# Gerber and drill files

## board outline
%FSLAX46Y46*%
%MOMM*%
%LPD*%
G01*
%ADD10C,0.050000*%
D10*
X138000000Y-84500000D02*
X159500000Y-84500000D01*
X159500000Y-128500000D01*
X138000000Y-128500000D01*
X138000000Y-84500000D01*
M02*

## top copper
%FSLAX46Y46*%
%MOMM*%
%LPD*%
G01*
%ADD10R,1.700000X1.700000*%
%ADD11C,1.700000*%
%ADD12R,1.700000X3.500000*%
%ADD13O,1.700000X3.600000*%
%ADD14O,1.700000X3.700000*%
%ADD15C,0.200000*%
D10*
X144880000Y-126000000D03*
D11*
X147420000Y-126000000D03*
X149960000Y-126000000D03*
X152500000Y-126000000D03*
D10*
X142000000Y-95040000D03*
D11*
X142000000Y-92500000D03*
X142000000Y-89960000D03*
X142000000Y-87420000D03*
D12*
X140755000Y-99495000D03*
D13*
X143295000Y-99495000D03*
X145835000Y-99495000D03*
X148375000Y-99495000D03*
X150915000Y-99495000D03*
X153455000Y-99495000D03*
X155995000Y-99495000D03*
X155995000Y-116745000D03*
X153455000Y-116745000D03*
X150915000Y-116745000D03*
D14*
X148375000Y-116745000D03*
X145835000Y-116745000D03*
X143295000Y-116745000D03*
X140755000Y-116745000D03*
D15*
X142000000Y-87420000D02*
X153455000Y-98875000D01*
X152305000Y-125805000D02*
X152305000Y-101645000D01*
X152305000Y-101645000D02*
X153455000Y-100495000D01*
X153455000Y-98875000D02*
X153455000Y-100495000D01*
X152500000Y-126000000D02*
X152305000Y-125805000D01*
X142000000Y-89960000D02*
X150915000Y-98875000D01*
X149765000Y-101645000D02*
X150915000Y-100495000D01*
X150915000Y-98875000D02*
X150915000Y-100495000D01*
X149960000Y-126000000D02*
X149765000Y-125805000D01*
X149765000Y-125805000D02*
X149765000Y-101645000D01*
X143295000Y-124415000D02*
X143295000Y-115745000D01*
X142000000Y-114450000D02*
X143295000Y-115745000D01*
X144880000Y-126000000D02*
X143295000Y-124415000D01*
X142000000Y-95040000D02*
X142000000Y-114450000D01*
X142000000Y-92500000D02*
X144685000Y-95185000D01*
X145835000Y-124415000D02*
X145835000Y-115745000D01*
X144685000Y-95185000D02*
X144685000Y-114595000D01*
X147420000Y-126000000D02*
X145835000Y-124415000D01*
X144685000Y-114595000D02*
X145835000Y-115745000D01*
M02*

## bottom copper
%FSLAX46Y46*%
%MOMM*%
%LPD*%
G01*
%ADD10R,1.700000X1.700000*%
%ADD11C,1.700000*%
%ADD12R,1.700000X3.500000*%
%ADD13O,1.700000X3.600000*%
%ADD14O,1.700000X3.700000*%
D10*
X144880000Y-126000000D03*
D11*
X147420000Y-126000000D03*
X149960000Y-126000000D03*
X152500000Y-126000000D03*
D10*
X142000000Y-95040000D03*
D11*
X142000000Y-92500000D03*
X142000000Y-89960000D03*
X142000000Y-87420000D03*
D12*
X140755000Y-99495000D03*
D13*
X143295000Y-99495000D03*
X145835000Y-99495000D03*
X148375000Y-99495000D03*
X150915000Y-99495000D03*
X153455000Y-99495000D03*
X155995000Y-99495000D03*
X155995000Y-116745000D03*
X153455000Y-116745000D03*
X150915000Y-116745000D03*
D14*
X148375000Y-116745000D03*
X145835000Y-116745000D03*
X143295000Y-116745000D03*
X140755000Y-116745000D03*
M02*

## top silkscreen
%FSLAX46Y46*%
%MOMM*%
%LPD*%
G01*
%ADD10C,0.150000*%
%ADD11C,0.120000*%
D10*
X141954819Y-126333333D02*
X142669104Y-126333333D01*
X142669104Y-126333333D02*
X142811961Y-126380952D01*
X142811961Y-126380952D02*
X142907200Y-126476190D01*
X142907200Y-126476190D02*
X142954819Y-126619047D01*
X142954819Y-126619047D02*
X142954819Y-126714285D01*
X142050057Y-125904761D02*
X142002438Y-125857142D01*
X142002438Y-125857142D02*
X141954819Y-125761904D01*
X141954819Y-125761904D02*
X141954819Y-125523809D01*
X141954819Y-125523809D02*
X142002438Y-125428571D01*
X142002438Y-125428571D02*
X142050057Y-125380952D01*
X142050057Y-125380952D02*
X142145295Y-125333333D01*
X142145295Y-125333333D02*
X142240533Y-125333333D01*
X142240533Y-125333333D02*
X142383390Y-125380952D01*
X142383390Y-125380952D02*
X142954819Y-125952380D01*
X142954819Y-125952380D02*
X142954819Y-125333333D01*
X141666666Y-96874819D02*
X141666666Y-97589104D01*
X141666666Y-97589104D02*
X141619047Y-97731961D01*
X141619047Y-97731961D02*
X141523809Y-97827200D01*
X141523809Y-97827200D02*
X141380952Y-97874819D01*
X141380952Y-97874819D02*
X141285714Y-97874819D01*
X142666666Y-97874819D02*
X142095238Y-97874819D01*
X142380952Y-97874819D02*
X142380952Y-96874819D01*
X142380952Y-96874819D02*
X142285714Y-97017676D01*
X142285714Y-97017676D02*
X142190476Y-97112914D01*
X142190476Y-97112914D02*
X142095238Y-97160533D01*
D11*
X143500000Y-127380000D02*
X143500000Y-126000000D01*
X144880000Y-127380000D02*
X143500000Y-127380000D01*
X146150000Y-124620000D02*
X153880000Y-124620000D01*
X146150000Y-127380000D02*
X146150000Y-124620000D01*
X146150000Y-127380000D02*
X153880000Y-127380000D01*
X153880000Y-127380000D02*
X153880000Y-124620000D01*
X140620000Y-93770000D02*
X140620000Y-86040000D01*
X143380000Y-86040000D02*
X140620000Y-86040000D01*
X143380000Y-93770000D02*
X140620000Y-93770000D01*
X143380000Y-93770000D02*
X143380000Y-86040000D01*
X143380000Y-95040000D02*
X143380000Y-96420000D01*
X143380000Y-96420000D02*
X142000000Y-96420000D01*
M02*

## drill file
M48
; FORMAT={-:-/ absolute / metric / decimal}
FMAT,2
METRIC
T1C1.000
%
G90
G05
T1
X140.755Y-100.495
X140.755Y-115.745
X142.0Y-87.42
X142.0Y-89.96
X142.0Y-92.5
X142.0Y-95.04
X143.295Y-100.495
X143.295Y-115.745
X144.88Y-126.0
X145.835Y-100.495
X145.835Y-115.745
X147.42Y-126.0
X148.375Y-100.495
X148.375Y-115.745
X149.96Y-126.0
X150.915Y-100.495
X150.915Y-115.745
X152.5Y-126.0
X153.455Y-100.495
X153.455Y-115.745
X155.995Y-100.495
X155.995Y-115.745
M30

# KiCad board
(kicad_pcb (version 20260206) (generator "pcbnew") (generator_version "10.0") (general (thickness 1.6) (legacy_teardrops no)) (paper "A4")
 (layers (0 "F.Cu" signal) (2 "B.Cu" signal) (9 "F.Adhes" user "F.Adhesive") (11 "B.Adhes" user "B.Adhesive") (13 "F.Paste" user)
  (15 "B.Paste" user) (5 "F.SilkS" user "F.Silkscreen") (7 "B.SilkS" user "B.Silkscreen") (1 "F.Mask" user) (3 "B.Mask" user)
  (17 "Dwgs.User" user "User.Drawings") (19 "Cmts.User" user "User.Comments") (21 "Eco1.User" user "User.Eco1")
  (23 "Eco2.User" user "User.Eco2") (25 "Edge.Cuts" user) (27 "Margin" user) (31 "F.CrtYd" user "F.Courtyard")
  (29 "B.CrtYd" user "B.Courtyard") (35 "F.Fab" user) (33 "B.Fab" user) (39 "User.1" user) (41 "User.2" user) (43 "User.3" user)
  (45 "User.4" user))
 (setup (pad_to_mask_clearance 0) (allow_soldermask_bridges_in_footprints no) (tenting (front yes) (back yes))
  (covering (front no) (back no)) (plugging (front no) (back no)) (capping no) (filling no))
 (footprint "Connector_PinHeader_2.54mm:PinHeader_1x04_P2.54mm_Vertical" (layer "F.Cu") (at 144.88 126 90)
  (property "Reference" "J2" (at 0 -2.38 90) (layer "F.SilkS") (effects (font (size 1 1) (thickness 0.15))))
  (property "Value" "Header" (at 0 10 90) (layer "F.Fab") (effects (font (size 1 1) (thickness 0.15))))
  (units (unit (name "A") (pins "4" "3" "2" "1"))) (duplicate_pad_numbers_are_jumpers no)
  (fp_line (start -1.38 -1.38) (end 0 -1.38) (stroke (width 0.12) (type solid)) (layer "F.SilkS"))
  (fp_line (start -1.38 0) (end -1.38 -1.38) (stroke (width 0.12) (type solid)) (layer "F.SilkS"))
  (fp_line (start 1.38 1.27) (end 1.38 9) (stroke (width 0.12) (type solid)) (layer "F.SilkS"))
  (fp_line (start -1.38 1.27) (end 1.38 1.27) (stroke (width 0.12) (type solid)) (layer "F.SilkS"))
  (fp_line (start -1.38 1.27) (end -1.38 9) (stroke (width 0.12) (type solid)) (layer "F.SilkS"))
  (fp_line (start -1.38 9) (end 1.38 9) (stroke (width 0.12) (type solid)) (layer "F.SilkS"))
  (pad "1" thru_hole rect (at 0 0 90) (size 1.7 1.7) (drill 1) (layers "*.Cu" "*.Mask") (remove_unused_layers no) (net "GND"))
  (pad "2" thru_hole circle (at 0 2.54 90) (size 1.7 1.7) (drill 1) (layers "*.Cu" "*.Mask") (remove_unused_layers no) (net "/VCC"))
  (pad "3" thru_hole circle (at 0 5.08 90) (size 1.7 1.7) (drill 1) (layers "*.Cu" "*.Mask") (remove_unused_layers no) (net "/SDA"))
  (pad "4" thru_hole circle (at 0 7.62 90) (size 1.7 1.7) (drill 1) (layers "*.Cu" "*.Mask") (remove_unused_layers no) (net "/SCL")))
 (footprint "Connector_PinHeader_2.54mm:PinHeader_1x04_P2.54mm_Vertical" (layer "F.Cu") (at 142 95.04 180)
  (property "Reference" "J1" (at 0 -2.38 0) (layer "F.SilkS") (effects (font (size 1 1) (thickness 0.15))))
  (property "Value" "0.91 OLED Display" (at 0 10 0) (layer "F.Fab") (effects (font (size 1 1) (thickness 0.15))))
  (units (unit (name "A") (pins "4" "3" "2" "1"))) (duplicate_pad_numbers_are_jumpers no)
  (fp_line (start 1.38 1.27) (end 1.38 9) (stroke (width 0.12) (type solid)) (layer "F.SilkS"))
  (fp_line (start -1.38 9) (end 1.38 9) (stroke (width 0.12) (type solid)) (layer "F.SilkS"))
  (fp_line (start -1.38 1.27) (end 1.38 1.27) (stroke (width 0.12) (type solid)) (layer "F.SilkS"))
  (fp_line (start -1.38 1.27) (end -1.38 9) (stroke (width 0.12) (type solid)) (layer "F.SilkS"))
  (fp_line (start -1.38 0) (end -1.38 -1.38) (stroke (width 0.12) (type solid)) (layer "F.SilkS"))
  (fp_line (start -1.38 -1.38) (end 0 -1.38) (stroke (width 0.12) (type solid)) (layer "F.SilkS"))
  (pad "1" thru_hole rect (at 0 0 180) (size 1.7 1.7) (drill 1) (layers "*.Cu" "*.Mask") (remove_unused_layers no) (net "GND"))
  (pad "2" thru_hole circle (at 0 2.54 180) (size 1.7 1.7) (drill 1) (layers "*.Cu" "*.Mask") (remove_unused_layers no) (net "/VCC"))
  (pad "3" thru_hole circle (at 0 5.08 180) (size 1.7 1.7) (drill 1) (layers "*.Cu" "*.Mask") (remove_unused_layers no) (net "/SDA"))
  (pad "4" thru_hole circle (at 0 7.62 180) (size 1.7 1.7) (drill 1) (layers "*.Cu" "*.Mask") (remove_unused_layers no) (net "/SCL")))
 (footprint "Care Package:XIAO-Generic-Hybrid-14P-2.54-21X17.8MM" (layer "B.Cu") (at 148.375 108.12 -90)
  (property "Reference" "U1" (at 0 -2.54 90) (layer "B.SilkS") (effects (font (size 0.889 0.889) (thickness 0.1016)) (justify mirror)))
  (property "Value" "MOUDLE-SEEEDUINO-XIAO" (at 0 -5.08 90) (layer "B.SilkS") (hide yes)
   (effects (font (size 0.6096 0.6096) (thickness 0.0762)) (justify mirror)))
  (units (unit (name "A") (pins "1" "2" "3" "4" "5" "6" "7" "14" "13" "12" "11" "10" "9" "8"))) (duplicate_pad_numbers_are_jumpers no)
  (pad "1" thru_hole rect (at -7.625 7.62 270) (size 3.5 1.7) (drill 1 (offset -1 0)) (layers "*.Cu" "*.Mask") (remove_unused_layers no)
   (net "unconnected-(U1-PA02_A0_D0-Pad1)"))
  (pad "2" thru_hole oval (at -7.625 5.08 270) (size 3.6 1.7) (drill 1 (offset -1 0)) (layers "*.Cu" "*.Mask") (remove_unused_layers no)
   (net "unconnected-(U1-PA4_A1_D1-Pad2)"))
  (pad "3" thru_hole oval (at -7.625 2.54 270) (size 3.6 1.7) (drill 1 (offset -1 0)) (layers "*.Cu" "*.Mask") (remove_unused_layers no)
   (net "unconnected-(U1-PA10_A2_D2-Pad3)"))
  (pad "4" thru_hole oval (at -7.625 0 270) (size 3.6 1.7) (drill 1 (offset -1 0)) (layers "*.Cu" "*.Mask") (remove_unused_layers no)
   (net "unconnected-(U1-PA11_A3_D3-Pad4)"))
  (pad "5" thru_hole oval (at -7.625 -2.54 270) (size 3.6 1.7) (drill 1 (offset -1 0)) (layers "*.Cu" "*.Mask") (remove_unused_layers no)
   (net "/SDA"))
  (pad "6" thru_hole oval (at -7.625 -5.08 90) (size 3.6 1.7) (drill 1 (offset 1 0)) (layers "*.Cu" "*.Mask") (remove_unused_layers no)
   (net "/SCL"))
  (pad "7" thru_hole oval (at -7.625 -7.62 270) (size 3.6 1.7) (drill 1 (offset -1 0)) (layers "*.Cu" "*.Mask") (remove_unused_layers no)
   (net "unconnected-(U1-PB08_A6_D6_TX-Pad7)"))
  (pad "8" thru_hole oval (at 7.625 -7.62 270) (size 3.6 1.7) (drill 1 (offset 1 0)) (layers "*.Cu" "*.Mask") (remove_unused_layers no)
   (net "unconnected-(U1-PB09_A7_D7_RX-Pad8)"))
  (pad "9" thru_hole oval (at 7.625 -5.08 270) (size 3.6 1.7) (drill 1 (offset 1 0)) (layers "*.Cu" "*.Mask") (remove_unused_layers no)
   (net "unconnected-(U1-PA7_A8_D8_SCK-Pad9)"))
  (pad "10" thru_hole oval (at 7.625 -2.54 270) (size 3.6 1.7) (drill 1 (offset 1 0)) (layers "*.Cu" "*.Mask") (remove_unused_layers no)
   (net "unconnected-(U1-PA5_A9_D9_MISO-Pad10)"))
  (pad "11" thru_hole oval (at 7.625 0 270) (size 3.7 1.7) (drill 1 (offset 1 0)) (layers "*.Cu" "*.Mask") (remove_unused_layers no)
   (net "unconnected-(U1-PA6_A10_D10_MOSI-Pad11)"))
  (pad "12" thru_hole oval (at 7.625 2.54 270) (size 3.7 1.7) (drill 1 (offset 1 0)) (layers "*.Cu" "*.Mask") (remove_unused_layers no)
   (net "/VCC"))
  (pad "13" thru_hole oval (at 7.625 5.08 270) (size 3.7 1.7) (drill 1 (offset 1 0)) (layers "*.Cu" "*.Mask") (remove_unused_layers no)
   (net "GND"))
  (pad "14" thru_hole oval (at 7.625 7.62 270) (size 3.7 1.7) (drill 1 (offset 1 0)) (layers "*.Cu" "*.Mask") (remove_unused_layers no)
   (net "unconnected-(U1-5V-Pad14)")))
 (gr_rect (start 138 84.5) (end 159.5 128.5) (stroke (width 0.05) (type default)) (fill no) (layer "Edge.Cuts"))
 (segment (start 142 87.42) (end 153.455 98.875) (width 0.2) (layer "F.Cu") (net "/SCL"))
 (segment (start 152.305 125.805) (end 152.305 101.645) (width 0.2) (layer "F.Cu") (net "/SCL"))
 (segment (start 152.305 101.645) (end 153.455 100.495) (width 0.2) (layer "F.Cu") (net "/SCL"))
 (segment (start 153.455 98.875) (end 153.455 100.495) (width 0.2) (layer "F.Cu") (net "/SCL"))
 (segment (start 152.5 126) (end 152.305 125.805) (width 0.2) (layer "F.Cu") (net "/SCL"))
 (segment (start 142 89.96) (end 150.915 98.875) (width 0.2) (layer "F.Cu") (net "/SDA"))
 (segment (start 149.765 101.645) (end 150.915 100.495) (width 0.2) (layer "F.Cu") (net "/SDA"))
 (segment (start 150.915 98.875) (end 150.915 100.495) (width 0.2) (layer "F.Cu") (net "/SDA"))
 (segment (start 149.96 126) (end 149.765 125.805) (width 0.2) (layer "F.Cu") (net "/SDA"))
 (segment (start 149.765 125.805) (end 149.765 101.645) (width 0.2) (layer "F.Cu") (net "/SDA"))
 (segment (start 143.295 124.415) (end 143.295 115.745) (width 0.2) (layer "F.Cu") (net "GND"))
 (segment (start 142 114.45) (end 143.295 115.745) (width 0.2) (layer "F.Cu") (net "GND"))
 (segment (start 144.88 126) (end 143.295 124.415) (width 0.2) (layer "F.Cu") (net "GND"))
 (segment (start 142 95.04) (end 142 114.45) (width 0.2) (layer "F.Cu") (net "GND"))
 (segment (start 142 92.5) (end 144.685 95.185) (width 0.2) (layer "F.Cu") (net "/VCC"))
 (segment (start 145.835 124.415) (end 145.835 115.745) (width 0.2) (layer "F.Cu") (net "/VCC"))
 (segment (start 144.685 95.185) (end 144.685 114.595) (width 0.2) (layer "F.Cu") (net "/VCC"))
 (segment (start 147.42 126) (end 145.835 124.415) (width 0.2) (layer "F.Cu") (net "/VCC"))
 (segment (start 144.685 114.595) (end 145.835 115.745) (width 0.2) (layer "F.Cu") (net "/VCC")))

